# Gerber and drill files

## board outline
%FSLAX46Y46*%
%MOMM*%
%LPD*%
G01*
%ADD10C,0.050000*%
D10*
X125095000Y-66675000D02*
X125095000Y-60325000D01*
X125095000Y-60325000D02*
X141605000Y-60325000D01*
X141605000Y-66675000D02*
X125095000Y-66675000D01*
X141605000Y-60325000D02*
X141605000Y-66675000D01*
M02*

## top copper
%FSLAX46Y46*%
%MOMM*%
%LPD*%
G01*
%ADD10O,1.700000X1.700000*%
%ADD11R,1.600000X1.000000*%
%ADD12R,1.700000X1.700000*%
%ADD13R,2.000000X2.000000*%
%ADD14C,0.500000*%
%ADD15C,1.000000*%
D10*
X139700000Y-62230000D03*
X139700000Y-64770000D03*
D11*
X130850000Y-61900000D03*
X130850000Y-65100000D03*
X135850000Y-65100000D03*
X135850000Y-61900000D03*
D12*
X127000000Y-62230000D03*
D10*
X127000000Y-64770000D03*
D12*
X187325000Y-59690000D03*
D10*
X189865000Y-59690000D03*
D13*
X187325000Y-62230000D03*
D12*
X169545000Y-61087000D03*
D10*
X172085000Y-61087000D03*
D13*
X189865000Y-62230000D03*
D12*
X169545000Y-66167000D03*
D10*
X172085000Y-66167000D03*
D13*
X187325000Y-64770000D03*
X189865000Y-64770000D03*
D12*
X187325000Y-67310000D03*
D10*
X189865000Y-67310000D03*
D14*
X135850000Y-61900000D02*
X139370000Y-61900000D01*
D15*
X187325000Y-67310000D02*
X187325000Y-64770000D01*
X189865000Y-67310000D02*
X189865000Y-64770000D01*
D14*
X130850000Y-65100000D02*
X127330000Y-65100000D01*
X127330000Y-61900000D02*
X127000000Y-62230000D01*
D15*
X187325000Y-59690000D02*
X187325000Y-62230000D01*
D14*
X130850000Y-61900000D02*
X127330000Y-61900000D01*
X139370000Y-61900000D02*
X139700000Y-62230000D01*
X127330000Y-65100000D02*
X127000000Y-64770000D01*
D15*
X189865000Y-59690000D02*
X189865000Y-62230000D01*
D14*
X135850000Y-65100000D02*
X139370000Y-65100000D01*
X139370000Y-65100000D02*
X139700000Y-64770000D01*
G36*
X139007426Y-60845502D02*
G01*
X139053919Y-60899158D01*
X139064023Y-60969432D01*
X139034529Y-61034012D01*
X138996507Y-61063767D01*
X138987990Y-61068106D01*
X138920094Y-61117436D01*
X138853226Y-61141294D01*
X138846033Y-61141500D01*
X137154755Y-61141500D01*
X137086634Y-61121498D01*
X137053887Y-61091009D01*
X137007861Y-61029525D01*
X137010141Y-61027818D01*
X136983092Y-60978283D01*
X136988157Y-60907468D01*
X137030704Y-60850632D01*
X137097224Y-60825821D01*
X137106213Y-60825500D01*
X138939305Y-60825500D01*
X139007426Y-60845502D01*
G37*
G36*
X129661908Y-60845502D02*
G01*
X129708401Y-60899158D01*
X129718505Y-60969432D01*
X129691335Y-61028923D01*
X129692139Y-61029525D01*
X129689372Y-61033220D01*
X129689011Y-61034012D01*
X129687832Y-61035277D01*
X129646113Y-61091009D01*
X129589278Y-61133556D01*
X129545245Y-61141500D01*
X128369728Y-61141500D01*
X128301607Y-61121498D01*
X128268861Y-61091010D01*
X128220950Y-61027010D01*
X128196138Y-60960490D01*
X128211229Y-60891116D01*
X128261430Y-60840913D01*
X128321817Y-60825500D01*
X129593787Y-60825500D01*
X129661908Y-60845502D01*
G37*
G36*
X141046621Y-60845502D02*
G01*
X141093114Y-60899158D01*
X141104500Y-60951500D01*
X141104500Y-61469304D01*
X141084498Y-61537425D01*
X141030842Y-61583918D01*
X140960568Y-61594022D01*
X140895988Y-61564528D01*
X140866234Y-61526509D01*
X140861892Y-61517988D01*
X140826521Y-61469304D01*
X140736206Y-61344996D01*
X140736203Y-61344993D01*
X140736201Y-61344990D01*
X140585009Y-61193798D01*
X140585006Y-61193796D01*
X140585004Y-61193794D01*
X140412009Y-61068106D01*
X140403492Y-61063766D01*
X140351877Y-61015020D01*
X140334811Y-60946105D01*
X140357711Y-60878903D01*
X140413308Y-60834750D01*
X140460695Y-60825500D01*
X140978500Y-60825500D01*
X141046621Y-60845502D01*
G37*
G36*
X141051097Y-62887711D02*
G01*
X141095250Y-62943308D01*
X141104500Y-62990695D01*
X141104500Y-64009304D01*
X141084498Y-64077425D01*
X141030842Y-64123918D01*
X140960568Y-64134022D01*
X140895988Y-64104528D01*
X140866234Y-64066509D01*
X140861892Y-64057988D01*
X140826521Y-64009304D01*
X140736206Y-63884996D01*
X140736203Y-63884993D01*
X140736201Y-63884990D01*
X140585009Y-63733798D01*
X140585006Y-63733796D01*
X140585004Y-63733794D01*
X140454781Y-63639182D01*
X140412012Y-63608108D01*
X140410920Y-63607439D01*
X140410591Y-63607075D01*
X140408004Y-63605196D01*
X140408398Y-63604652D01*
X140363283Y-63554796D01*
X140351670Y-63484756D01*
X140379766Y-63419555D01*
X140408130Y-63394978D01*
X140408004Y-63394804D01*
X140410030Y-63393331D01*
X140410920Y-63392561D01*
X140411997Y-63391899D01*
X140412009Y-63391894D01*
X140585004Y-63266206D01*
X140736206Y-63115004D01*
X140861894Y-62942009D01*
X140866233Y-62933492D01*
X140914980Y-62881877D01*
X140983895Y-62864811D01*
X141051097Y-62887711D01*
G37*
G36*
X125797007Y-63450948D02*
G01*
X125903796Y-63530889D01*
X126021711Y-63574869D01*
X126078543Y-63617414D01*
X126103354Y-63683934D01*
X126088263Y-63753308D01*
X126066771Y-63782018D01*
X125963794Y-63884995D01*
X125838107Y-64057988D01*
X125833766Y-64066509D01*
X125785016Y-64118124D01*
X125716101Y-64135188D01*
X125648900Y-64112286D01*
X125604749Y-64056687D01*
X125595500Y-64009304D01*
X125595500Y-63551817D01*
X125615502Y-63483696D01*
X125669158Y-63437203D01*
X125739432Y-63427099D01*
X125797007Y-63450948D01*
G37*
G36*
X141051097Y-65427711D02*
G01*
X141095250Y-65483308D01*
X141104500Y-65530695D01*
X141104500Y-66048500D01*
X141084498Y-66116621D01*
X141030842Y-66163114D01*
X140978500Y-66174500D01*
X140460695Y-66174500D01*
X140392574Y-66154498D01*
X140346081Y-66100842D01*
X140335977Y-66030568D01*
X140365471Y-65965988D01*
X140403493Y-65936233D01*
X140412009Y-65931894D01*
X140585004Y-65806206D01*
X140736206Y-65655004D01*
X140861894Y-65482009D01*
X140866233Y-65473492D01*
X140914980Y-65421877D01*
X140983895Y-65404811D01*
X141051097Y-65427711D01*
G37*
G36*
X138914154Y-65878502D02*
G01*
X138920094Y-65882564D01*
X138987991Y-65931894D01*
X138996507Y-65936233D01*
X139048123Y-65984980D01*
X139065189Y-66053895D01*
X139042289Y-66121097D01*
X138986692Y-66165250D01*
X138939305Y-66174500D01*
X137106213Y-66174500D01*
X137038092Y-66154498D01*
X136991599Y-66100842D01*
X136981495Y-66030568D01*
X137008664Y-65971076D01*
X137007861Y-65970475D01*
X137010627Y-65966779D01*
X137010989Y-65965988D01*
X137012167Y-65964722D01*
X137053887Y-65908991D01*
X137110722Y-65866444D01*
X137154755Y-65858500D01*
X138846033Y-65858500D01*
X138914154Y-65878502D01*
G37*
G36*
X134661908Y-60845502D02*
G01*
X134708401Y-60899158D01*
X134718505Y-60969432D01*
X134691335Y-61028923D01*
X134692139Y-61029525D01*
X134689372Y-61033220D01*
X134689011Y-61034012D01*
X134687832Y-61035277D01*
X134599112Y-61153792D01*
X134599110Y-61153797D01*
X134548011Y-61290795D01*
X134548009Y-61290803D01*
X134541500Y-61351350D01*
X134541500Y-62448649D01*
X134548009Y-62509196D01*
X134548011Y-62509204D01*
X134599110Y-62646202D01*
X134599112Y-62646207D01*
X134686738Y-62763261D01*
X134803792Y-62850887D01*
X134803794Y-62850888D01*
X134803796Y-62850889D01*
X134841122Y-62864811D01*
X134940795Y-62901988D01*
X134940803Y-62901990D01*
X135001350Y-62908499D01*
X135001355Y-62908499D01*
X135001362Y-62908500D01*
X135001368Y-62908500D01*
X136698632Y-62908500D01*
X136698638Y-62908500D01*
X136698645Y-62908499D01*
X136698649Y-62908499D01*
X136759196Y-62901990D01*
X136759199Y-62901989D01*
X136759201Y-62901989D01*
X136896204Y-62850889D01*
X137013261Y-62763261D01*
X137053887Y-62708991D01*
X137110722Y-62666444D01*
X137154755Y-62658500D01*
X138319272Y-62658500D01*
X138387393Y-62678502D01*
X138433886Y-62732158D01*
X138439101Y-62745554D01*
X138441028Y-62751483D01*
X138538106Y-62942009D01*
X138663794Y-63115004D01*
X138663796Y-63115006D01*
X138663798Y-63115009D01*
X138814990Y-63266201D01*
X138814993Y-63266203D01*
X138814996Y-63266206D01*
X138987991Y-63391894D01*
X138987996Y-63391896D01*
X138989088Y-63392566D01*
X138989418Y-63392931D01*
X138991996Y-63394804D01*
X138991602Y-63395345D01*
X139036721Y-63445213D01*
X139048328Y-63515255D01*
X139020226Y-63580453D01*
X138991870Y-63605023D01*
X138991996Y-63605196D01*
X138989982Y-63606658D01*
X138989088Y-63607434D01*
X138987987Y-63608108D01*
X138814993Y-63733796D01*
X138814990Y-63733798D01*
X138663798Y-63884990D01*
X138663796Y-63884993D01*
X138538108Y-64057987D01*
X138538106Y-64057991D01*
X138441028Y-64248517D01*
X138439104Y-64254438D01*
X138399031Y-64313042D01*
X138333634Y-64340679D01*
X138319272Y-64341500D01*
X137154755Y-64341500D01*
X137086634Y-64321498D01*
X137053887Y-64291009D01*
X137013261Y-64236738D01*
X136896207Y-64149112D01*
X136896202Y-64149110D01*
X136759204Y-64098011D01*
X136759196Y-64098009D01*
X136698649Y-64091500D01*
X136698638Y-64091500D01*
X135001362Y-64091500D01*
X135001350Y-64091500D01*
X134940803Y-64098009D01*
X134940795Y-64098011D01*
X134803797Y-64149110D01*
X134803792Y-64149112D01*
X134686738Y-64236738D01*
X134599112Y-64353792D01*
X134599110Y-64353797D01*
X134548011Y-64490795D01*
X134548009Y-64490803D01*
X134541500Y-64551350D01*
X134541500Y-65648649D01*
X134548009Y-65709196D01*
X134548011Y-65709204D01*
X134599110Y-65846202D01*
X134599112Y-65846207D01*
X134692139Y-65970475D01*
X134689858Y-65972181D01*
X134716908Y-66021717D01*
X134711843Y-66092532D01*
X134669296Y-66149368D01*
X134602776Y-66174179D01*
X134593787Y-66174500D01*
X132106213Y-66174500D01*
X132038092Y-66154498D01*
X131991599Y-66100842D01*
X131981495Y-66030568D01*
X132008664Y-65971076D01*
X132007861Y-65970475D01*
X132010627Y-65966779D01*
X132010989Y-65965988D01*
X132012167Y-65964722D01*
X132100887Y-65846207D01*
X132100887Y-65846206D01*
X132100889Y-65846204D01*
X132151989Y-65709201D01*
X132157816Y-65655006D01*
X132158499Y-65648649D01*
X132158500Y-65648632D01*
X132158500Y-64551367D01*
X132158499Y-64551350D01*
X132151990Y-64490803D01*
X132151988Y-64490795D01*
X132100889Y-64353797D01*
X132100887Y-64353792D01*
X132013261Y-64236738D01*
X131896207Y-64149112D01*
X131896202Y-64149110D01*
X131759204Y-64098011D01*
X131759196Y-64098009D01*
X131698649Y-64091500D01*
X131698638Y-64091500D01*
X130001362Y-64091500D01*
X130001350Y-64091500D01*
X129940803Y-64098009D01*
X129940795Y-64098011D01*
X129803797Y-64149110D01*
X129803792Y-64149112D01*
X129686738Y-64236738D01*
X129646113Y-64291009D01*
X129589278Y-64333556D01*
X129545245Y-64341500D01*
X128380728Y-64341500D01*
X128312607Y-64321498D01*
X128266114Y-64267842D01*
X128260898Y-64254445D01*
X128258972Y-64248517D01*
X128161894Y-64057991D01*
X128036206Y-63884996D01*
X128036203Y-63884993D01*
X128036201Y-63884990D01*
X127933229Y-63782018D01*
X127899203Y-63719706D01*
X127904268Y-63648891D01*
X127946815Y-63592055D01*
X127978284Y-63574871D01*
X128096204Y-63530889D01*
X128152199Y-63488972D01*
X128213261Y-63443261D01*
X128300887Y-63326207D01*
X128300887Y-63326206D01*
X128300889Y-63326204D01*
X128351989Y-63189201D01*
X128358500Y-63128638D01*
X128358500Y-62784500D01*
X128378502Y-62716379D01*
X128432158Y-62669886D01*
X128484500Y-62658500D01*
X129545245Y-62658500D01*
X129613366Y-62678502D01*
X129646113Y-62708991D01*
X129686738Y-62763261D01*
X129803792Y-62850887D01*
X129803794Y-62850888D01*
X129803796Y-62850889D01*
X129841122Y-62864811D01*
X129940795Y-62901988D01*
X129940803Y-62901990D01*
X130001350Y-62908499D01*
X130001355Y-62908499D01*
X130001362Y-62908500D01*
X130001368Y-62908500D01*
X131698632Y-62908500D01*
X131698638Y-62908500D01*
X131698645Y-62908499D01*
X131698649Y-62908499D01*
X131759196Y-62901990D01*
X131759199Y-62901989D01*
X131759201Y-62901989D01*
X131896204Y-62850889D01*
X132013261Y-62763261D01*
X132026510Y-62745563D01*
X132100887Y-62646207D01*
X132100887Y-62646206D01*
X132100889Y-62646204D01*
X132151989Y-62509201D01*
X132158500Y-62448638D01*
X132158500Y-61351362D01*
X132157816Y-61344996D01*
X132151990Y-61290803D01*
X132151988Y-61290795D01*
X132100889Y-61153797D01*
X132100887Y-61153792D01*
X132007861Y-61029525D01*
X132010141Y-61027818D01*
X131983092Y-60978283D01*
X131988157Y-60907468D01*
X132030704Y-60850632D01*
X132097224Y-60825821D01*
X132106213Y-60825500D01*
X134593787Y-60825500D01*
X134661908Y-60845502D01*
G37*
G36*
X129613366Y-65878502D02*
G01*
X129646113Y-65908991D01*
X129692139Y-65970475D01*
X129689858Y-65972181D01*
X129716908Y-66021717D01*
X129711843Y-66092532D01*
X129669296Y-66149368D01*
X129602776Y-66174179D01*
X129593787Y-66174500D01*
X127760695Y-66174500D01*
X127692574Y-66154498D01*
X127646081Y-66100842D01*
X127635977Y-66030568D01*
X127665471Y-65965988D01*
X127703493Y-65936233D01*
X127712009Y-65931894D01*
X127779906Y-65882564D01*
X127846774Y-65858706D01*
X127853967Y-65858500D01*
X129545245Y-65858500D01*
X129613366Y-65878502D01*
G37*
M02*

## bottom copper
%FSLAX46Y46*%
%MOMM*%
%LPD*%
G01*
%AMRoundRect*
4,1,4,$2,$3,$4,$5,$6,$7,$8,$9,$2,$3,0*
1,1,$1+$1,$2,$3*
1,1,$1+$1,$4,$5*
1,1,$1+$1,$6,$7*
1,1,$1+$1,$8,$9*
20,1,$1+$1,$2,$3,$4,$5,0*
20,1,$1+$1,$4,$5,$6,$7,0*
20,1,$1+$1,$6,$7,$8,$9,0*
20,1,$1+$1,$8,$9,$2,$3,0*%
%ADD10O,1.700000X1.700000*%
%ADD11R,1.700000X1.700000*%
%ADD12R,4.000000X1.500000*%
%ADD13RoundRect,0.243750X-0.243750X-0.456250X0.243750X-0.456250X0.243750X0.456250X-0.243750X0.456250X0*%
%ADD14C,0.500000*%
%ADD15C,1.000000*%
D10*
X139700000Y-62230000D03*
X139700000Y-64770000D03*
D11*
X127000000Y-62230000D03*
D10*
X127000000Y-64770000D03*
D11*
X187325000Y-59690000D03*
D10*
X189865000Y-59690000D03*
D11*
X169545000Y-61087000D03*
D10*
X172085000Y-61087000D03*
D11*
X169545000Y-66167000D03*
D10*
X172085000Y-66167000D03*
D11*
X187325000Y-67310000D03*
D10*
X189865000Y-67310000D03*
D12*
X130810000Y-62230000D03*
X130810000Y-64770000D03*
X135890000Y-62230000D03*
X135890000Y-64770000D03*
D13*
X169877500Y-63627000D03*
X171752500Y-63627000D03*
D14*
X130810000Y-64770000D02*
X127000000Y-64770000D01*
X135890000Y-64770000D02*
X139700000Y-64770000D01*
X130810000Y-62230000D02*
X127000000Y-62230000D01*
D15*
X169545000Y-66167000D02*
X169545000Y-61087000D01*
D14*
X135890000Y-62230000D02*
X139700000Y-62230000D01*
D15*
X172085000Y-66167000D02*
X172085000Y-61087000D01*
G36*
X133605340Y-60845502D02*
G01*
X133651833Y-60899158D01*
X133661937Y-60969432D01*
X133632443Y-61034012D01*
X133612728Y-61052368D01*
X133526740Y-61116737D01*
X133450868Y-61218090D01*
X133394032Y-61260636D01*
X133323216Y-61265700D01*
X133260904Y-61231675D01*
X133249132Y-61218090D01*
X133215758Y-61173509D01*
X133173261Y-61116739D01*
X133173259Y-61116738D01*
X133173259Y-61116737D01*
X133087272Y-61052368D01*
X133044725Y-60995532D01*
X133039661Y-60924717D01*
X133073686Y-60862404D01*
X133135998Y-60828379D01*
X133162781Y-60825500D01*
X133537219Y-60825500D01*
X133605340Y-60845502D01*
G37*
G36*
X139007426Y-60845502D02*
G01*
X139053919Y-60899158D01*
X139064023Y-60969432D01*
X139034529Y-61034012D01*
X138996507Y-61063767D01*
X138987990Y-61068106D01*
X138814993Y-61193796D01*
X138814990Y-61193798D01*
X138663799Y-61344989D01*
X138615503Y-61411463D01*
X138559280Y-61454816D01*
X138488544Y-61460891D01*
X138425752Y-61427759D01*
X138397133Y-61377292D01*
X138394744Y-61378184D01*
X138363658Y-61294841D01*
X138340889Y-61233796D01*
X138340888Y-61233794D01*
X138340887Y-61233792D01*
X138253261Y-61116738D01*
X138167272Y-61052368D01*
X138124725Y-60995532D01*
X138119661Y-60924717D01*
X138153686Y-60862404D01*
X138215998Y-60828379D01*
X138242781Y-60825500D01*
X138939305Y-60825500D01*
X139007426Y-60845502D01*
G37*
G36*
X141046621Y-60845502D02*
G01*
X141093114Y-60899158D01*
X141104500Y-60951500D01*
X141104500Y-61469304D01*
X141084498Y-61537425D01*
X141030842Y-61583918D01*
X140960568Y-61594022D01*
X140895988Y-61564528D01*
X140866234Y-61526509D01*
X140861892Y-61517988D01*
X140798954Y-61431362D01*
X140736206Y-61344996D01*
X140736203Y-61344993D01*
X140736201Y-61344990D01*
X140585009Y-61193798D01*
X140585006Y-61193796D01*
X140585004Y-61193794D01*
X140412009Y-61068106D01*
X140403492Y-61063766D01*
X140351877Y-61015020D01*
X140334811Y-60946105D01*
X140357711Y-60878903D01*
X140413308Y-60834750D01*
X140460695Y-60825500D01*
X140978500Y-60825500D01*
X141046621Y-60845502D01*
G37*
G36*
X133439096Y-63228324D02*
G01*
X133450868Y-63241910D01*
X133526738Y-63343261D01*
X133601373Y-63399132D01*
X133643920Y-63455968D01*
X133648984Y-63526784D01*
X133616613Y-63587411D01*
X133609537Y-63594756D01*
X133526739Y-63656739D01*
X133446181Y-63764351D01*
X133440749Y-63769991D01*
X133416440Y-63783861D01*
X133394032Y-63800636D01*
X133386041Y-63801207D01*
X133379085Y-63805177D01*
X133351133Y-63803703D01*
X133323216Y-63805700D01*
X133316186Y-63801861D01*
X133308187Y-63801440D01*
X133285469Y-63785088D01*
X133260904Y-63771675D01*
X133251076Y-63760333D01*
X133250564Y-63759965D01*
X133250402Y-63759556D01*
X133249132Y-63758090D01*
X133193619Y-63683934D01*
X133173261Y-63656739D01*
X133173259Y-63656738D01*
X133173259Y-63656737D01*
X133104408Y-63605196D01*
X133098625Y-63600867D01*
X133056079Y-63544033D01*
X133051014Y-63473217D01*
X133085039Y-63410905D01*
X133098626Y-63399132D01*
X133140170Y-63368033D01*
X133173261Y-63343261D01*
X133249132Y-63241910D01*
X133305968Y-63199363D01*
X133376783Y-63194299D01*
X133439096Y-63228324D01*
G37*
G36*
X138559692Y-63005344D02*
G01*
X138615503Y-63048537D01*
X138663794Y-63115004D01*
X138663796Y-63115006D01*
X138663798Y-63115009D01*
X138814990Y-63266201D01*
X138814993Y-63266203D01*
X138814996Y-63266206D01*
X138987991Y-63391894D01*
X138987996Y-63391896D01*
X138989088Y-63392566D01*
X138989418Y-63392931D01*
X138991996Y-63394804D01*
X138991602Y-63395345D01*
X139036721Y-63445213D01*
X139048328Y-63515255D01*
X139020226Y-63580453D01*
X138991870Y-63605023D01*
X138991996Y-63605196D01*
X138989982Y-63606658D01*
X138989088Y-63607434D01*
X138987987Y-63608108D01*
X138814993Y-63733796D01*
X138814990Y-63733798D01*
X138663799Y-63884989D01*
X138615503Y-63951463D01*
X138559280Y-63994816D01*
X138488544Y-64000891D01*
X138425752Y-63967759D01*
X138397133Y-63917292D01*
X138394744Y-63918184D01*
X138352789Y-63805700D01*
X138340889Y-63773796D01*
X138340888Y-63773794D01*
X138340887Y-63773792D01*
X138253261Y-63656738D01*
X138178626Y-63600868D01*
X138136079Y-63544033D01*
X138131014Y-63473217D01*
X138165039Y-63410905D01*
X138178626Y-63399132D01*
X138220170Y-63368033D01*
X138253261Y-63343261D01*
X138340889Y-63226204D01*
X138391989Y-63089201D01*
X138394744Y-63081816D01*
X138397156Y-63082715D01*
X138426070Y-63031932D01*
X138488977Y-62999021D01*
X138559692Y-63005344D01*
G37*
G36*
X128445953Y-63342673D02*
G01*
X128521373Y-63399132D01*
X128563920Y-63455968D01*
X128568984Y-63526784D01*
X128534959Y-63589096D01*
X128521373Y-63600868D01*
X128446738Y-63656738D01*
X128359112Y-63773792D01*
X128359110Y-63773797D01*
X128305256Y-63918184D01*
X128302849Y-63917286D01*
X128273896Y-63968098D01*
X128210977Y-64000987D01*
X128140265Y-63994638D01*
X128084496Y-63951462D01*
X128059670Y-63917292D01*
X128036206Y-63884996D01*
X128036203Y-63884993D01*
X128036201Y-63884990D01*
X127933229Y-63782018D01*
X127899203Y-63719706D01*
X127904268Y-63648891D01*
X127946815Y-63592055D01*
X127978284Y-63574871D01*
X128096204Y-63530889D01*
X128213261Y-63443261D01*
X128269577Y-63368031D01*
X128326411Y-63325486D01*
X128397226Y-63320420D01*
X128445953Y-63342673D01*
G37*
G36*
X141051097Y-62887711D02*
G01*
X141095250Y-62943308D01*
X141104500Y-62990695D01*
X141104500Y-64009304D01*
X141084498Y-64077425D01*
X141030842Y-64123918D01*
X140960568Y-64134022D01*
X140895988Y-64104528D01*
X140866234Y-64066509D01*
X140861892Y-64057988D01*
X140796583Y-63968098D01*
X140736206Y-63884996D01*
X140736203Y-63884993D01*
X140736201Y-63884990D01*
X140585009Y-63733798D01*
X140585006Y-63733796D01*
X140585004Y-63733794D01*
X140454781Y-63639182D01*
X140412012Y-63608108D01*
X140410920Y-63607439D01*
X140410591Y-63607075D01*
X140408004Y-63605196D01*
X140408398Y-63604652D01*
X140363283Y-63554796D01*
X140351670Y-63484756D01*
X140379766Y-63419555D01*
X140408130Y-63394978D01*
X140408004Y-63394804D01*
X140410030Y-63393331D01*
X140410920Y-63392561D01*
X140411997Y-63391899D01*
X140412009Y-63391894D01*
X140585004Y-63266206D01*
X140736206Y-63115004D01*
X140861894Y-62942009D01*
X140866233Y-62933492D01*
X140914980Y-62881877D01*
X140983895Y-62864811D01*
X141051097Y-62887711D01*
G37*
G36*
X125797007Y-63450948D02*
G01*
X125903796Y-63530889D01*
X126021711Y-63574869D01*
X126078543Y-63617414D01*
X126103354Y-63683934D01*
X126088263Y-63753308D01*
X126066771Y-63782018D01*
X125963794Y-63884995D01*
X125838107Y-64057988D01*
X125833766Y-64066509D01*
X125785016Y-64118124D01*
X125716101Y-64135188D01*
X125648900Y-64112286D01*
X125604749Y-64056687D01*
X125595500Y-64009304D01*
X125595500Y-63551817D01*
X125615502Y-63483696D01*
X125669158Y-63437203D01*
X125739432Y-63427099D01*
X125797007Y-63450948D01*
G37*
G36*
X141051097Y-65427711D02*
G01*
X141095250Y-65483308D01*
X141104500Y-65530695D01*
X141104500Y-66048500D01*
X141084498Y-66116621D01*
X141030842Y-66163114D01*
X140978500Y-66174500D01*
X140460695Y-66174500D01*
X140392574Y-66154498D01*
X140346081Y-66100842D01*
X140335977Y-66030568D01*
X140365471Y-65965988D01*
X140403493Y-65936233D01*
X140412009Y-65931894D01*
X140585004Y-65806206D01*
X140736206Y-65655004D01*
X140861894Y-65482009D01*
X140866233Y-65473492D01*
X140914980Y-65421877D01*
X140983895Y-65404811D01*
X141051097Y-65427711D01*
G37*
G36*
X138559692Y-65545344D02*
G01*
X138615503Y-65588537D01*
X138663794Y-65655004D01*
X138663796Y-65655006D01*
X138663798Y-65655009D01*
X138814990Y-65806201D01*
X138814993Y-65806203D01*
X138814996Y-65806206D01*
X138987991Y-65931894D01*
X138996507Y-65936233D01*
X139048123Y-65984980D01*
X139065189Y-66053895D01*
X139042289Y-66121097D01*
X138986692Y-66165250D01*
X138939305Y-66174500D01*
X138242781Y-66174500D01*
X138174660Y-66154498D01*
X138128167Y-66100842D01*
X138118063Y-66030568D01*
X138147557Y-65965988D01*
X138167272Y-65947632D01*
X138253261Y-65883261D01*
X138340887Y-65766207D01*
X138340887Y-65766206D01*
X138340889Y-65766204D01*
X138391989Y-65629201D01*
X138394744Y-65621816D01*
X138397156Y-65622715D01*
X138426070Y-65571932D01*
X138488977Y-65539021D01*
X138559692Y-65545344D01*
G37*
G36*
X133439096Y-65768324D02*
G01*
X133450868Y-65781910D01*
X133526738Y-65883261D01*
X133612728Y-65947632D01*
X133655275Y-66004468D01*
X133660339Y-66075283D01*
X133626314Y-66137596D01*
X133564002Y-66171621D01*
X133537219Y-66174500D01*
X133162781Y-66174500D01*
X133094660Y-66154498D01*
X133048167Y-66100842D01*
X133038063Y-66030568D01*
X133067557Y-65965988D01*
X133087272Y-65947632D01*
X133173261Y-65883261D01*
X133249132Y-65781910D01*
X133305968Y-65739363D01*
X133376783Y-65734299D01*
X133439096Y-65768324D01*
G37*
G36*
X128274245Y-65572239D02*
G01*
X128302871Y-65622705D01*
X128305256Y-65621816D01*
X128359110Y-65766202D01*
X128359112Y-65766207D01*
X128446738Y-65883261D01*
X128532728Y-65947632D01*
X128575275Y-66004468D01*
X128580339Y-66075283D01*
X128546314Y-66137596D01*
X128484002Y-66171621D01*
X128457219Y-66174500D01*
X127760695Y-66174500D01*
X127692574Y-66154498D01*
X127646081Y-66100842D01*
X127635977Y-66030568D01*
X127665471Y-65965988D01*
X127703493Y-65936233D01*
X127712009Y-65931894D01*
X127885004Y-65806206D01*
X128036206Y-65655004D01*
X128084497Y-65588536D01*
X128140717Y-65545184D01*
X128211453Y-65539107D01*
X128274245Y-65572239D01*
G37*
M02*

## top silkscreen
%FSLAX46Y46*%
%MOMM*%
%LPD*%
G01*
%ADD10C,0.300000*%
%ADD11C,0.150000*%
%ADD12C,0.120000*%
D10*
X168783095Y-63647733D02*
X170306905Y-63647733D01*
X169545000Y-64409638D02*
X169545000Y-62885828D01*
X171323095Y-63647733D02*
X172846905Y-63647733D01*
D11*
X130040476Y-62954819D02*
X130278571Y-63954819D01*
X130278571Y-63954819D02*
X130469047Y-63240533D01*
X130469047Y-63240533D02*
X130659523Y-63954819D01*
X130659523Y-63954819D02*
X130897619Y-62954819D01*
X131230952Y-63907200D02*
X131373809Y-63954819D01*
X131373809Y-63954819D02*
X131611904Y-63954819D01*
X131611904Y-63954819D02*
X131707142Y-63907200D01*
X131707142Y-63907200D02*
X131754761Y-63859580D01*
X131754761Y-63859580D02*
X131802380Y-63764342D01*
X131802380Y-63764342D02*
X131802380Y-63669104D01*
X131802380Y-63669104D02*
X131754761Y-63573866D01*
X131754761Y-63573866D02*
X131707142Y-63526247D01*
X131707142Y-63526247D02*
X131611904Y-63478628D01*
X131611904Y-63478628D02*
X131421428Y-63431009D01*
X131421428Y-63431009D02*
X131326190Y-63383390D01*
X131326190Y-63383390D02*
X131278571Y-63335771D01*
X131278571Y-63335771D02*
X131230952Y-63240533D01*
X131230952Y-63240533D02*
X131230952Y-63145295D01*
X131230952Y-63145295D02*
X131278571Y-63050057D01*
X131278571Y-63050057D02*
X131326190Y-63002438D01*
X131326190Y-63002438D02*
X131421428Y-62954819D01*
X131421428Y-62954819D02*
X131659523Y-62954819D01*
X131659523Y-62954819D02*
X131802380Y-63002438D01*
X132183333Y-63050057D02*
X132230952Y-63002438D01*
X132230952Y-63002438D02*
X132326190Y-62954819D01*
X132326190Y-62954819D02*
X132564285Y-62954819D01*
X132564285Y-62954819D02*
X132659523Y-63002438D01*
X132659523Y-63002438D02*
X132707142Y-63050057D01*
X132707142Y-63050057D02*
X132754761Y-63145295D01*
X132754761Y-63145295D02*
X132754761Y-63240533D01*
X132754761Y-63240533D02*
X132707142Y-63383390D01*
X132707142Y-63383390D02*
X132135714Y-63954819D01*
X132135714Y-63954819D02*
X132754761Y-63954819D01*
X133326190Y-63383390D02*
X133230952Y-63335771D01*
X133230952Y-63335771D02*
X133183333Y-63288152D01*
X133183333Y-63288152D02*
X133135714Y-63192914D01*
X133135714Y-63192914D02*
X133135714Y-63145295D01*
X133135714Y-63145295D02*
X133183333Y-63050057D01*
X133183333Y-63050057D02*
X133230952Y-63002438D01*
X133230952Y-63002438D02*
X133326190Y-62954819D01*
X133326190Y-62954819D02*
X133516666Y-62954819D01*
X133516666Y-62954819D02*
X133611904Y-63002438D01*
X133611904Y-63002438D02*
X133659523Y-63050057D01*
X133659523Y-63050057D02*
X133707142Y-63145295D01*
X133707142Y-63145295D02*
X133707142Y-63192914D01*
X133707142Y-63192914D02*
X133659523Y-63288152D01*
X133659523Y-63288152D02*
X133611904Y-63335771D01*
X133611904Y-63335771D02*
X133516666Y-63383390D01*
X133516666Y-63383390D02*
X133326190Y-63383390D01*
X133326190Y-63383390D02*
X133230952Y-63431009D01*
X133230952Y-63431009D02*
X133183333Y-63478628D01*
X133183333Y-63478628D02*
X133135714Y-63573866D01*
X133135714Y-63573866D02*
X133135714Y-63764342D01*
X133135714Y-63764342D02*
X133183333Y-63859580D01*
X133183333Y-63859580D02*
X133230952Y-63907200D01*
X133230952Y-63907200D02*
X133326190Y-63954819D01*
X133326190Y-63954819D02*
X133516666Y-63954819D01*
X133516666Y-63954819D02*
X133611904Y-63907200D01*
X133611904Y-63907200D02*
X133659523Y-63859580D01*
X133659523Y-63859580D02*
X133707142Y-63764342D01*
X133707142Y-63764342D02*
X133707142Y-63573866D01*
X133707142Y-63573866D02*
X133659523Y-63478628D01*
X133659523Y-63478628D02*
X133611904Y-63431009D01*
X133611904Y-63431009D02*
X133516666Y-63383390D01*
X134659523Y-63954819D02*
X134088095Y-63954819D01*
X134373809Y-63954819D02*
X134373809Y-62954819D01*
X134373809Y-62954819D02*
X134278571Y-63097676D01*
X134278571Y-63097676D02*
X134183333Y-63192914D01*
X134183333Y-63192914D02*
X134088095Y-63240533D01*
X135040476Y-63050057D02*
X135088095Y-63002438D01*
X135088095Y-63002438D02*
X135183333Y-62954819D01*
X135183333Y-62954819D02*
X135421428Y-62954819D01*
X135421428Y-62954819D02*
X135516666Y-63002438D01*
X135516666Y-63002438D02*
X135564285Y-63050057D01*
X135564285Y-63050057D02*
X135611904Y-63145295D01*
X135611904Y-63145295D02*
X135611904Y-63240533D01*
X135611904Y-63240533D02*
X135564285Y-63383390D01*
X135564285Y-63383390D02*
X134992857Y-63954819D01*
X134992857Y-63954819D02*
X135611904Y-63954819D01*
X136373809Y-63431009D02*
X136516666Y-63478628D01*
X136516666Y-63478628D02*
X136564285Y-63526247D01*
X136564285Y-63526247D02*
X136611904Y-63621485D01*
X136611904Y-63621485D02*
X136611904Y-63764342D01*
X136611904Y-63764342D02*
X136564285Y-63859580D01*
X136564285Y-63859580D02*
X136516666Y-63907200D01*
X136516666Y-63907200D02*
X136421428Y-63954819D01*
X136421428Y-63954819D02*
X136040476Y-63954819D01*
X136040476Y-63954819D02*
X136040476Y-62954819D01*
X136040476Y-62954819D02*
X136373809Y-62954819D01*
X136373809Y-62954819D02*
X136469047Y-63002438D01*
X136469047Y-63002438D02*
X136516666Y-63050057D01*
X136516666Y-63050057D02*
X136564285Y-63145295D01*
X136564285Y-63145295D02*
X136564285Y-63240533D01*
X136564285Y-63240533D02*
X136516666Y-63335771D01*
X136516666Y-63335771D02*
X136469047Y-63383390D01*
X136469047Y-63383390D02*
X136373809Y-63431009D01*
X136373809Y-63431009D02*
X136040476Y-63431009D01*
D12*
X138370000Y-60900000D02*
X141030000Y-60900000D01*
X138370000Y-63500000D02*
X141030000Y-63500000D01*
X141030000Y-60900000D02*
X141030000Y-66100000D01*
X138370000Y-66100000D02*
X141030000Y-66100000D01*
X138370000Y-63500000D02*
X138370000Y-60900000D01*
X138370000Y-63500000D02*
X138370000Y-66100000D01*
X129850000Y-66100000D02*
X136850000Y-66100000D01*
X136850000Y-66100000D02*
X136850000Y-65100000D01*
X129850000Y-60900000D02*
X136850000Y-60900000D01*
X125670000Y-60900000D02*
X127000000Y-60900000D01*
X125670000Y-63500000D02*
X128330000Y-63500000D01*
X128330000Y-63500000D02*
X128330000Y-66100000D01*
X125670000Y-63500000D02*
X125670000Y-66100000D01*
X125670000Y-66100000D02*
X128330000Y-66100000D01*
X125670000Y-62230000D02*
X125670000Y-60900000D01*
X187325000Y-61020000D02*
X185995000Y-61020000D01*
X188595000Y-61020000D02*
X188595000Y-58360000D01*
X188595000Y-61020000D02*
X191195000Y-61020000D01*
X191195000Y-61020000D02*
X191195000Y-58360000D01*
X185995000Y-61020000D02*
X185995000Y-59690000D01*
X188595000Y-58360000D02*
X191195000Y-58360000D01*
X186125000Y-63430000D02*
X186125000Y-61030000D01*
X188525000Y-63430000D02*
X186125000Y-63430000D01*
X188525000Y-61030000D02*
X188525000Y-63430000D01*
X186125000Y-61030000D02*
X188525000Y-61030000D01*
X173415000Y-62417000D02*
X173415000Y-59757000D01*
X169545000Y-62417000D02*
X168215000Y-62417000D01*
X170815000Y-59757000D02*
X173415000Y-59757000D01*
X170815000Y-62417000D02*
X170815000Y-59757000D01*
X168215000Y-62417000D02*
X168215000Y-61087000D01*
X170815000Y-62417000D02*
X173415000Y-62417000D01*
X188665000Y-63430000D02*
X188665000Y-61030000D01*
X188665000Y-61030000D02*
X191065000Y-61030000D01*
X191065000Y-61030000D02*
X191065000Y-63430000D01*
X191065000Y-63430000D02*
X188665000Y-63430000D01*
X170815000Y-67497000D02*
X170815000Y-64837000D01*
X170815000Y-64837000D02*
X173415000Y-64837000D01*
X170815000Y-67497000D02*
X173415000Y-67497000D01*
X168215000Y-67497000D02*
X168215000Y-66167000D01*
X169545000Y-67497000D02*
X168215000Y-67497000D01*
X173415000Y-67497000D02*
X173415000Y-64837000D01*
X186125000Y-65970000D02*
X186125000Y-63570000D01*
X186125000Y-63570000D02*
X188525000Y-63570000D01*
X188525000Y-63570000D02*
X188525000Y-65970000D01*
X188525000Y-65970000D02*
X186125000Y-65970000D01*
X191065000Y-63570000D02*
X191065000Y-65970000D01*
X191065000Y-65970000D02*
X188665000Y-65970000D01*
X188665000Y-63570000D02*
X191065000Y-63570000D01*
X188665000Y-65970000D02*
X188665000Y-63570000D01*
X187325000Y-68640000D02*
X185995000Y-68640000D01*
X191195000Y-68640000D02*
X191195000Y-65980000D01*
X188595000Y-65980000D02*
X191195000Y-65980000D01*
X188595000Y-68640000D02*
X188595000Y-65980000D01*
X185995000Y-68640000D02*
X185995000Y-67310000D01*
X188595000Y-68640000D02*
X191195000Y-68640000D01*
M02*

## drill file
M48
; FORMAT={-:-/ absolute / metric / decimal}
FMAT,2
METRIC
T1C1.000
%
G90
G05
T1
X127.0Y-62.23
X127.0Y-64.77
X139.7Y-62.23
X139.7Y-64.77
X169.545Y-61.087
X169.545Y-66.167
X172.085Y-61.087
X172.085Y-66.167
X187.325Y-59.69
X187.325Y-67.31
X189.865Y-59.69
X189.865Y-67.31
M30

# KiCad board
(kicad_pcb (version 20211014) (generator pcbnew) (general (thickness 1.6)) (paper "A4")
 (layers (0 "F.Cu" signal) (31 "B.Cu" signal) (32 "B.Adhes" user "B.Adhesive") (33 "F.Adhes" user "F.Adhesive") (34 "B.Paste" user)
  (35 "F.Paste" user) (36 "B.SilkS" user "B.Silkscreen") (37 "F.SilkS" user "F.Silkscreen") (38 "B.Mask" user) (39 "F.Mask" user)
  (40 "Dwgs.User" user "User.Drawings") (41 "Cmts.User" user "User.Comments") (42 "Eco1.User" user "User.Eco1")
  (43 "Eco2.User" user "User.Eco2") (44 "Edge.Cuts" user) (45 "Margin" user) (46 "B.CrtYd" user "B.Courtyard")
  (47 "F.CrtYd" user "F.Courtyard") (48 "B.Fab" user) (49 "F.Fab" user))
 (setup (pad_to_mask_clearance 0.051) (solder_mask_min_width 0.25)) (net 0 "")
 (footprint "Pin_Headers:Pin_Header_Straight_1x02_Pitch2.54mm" (layer "F.Cu") (at 139.7 62.23)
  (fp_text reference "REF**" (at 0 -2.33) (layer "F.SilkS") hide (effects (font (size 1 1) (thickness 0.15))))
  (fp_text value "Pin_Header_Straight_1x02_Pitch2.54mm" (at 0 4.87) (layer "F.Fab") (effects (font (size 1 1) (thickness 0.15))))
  (fp_line (start -1.33 -1.33) (end 1.33 -1.33) (layer "F.SilkS") (width 0.12))
  (fp_line (start -1.33 1.27) (end 1.33 1.27) (layer "F.SilkS") (width 0.12))
  (fp_line (start 1.33 -1.33) (end 1.33 3.87) (layer "F.SilkS") (width 0.12))
  (fp_line (start -1.33 3.87) (end 1.33 3.87) (layer "F.SilkS") (width 0.12))
  (fp_line (start -1.33 1.27) (end -1.33 -1.33) (layer "F.SilkS") (width 0.12))
  (fp_line (start -1.33 1.27) (end -1.33 3.87) (layer "F.SilkS") (width 0.12))
  (pad "1" thru_hole oval locked (at 0 0) (size 1.7 1.7) (drill 1) (layers *.Cu *.Mask))
  (pad "2" thru_hole oval locked (at 0 2.54) (size 1.7 1.7) (drill 1) (layers *.Cu *.Mask)))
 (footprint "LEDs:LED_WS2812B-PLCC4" (layer "F.Cu") (at 133.35 63.5)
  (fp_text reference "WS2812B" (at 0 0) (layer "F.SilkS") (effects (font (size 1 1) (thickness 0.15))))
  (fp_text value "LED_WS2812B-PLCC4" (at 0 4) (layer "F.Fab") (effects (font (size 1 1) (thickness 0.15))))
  (fp_line (start -3.5 2.6) (end 3.5 2.6) (layer "F.SilkS") (width 0.12))
  (fp_line (start 3.5 2.6) (end 3.5 1.6) (layer "F.SilkS") (width 0.12))
  (fp_line (start -3.5 -2.6) (end 3.5 -2.6) (layer "F.SilkS") (width 0.12))
  (pad "1" smd rect locked (at -2.5 -1.6) (size 1.6 1) (layers "F.Cu" "F.Paste" "F.Mask"))
  (pad "2" smd rect locked (at -2.5 1.6) (size 1.6 1) (layers "F.Cu" "F.Paste" "F.Mask"))
  (pad "3" smd rect locked (at 2.5 1.6) (size 1.6 1) (layers "F.Cu" "F.Paste" "F.Mask"))
  (pad "4" smd rect locked (at 2.5 -1.6) (size 1.6 1) (layers "F.Cu" "F.Paste" "F.Mask")))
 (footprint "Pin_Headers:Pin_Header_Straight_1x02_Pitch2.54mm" (layer "F.Cu") (at 127 62.23)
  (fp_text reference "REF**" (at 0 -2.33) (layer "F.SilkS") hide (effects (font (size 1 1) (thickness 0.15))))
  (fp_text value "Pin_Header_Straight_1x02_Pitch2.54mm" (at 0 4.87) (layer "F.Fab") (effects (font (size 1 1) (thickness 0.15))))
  (fp_line (start -1.33 -1.33) (end 0 -1.33) (layer "F.SilkS") (width 0.12))
  (fp_line (start -1.33 1.27) (end 1.33 1.27) (layer "F.SilkS") (width 0.12))
  (fp_line (start 1.33 1.27) (end 1.33 3.87) (layer "F.SilkS") (width 0.12))
  (fp_line (start -1.33 1.27) (end -1.33 3.87) (layer "F.SilkS") (width 0.12))
  (fp_line (start -1.33 3.87) (end 1.33 3.87) (layer "F.SilkS") (width 0.12))
  (fp_line (start -1.33 0) (end -1.33 -1.33) (layer "F.SilkS") (width 0.12))
  (pad "1" thru_hole rect locked (at 0 0) (size 1.7 1.7) (drill 1) (layers *.Cu *.Mask))
  (pad "2" thru_hole oval locked (at 0 2.54) (size 1.7 1.7) (drill 1) (layers *.Cu *.Mask)))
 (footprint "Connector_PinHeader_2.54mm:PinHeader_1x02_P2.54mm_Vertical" (layer "F.Cu") (at 187.325 59.69 90)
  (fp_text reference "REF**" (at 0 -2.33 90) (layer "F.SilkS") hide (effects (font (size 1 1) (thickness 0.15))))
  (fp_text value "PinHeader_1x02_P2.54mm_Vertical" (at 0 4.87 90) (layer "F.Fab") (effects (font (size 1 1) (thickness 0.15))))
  (fp_line (start -1.33 0) (end -1.33 -1.33) (layer "F.SilkS") (width 0.12))
  (fp_line (start -1.33 1.27) (end 1.33 1.27) (layer "F.SilkS") (width 0.12))
  (fp_line (start -1.33 1.27) (end -1.33 3.87) (layer "F.SilkS") (width 0.12))
  (fp_line (start -1.33 3.87) (end 1.33 3.87) (layer "F.SilkS") (width 0.12))
  (fp_line (start -1.33 -1.33) (end 0 -1.33) (layer "F.SilkS") (width 0.12))
  (fp_line (start 1.33 1.27) (end 1.33 3.87) (layer "F.SilkS") (width 0.12))
  (pad "1" thru_hole rect locked (at 0 0 90) (size 1.7 1.7) (drill 1) (layers *.Cu *.Mask))
  (pad "2" thru_hole oval locked (at 0 2.54 90) (size 1.7 1.7) (drill 1) (layers *.Cu *.Mask)))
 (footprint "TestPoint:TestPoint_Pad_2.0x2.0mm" (layer "F.Cu") (at 187.325 62.23)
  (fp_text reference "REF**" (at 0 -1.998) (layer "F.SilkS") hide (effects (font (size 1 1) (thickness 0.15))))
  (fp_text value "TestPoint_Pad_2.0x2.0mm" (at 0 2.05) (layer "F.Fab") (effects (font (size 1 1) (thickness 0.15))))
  (fp_line (start -1.2 1.2) (end -1.2 -1.2) (layer "F.SilkS") (width 0.12))
  (fp_line (start 1.2 1.2) (end -1.2 1.2) (layer "F.SilkS") (width 0.12))
  (fp_line (start 1.2 -1.2) (end 1.2 1.2) (layer "F.SilkS") (width 0.12))
  (fp_line (start -1.2 -1.2) (end 1.2 -1.2) (layer "F.SilkS") (width 0.12))
  (pad "1" smd rect locked (at 0 0) (size 2 2) (layers "F.Cu" "F.Mask")))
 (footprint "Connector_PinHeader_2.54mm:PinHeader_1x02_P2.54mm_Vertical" (layer "F.Cu") (at 169.545 61.087 90)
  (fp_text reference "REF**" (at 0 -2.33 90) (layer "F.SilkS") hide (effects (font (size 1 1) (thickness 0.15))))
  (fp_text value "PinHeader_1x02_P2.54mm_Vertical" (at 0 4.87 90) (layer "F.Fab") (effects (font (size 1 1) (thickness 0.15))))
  (fp_line (start -1.33 3.87) (end 1.33 3.87) (layer "F.SilkS") (width 0.12))
  (fp_line (start -1.33 0) (end -1.33 -1.33) (layer "F.SilkS") (width 0.12))
  (fp_line (start 1.33 1.27) (end 1.33 3.87) (layer "F.SilkS") (width 0.12))
  (fp_line (start -1.33 1.27) (end 1.33 1.27) (layer "F.SilkS") (width 0.12))
  (fp_line (start -1.33 -1.33) (end 0 -1.33) (layer "F.SilkS") (width 0.12))
  (fp_line (start -1.33 1.27) (end -1.33 3.87) (layer "F.SilkS") (width 0.12))
  (pad "1" thru_hole rect locked (at 0 0 90) (size 1.7 1.7) (drill 1) (layers *.Cu *.Mask))
  (pad "2" thru_hole oval locked (at 0 2.54 90) (size 1.7 1.7) (drill 1) (layers *.Cu *.Mask)))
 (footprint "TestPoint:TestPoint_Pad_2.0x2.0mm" (layer "F.Cu") (at 189.865 62.23)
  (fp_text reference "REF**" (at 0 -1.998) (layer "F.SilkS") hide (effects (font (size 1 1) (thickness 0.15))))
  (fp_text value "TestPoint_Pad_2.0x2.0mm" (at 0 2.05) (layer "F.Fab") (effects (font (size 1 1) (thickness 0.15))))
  (fp_line (start -1.2 1.2) (end -1.2 -1.2) (layer "F.SilkS") (width 0.12))
  (fp_line (start -1.2 -1.2) (end 1.2 -1.2) (layer "F.SilkS") (width 0.12))
  (fp_line (start 1.2 -1.2) (end 1.2 1.2) (layer "F.SilkS") (width 0.12))
  (fp_line (start 1.2 1.2) (end -1.2 1.2) (layer "F.SilkS") (width 0.12))
  (pad "1" smd rect locked (at 0 0) (size 2 2) (layers "F.Cu" "F.Mask")))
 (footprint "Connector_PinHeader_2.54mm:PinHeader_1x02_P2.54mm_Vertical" (layer "F.Cu") (at 169.545 66.167 90)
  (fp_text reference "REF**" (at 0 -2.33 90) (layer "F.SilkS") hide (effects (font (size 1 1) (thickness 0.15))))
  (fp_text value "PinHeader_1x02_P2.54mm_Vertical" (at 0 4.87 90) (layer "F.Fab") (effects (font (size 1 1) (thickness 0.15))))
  (fp_line (start -1.33 1.27) (end 1.33 1.27) (layer "F.SilkS") (width 0.12))
  (fp_line (start 1.33 1.27) (end 1.33 3.87) (layer "F.SilkS") (width 0.12))
  (fp_line (start -1.33 1.27) (end -1.33 3.87) (layer "F.SilkS") (width 0.12))
  (fp_line (start -1.33 -1.33) (end 0 -1.33) (layer "F.SilkS") (width 0.12))
  (fp_line (start -1.33 0) (end -1.33 -1.33) (layer "F.SilkS") (width 0.12))
  (fp_line (start -1.33 3.87) (end 1.33 3.87) (layer "F.SilkS") (width 0.12))
  (pad "1" thru_hole rect locked (at 0 0 90) (size 1.7 1.7) (drill 1) (layers *.Cu *.Mask))
  (pad "2" thru_hole oval locked (at 0 2.54 90) (size 1.7 1.7) (drill 1) (layers *.Cu *.Mask)))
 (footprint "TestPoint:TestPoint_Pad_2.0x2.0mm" (layer "F.Cu") (at 187.325 64.77)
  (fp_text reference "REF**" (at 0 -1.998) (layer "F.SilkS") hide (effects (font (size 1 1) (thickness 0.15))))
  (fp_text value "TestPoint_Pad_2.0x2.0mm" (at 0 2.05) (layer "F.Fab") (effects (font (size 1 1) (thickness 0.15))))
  (fp_line (start -1.2 1.2) (end -1.2 -1.2) (layer "F.SilkS") (width 0.12))
  (fp_line (start -1.2 -1.2) (end 1.2 -1.2) (layer "F.SilkS") (width 0.12))
  (fp_line (start 1.2 -1.2) (end 1.2 1.2) (layer "F.SilkS") (width 0.12))
  (fp_line (start 1.2 1.2) (end -1.2 1.2) (layer "F.SilkS") (width 0.12))
  (pad "1" smd rect locked (at 0 0) (size 2 2) (layers "F.Cu" "F.Mask")))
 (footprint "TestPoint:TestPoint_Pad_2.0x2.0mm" (layer "F.Cu") (at 189.865 64.77)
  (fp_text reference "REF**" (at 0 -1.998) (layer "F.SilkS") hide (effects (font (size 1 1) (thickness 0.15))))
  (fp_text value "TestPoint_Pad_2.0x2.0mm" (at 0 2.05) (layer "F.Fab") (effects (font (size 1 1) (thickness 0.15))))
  (fp_line (start 1.2 -1.2) (end 1.2 1.2) (layer "F.SilkS") (width 0.12))
  (fp_line (start 1.2 1.2) (end -1.2 1.2) (layer "F.SilkS") (width 0.12))
  (fp_line (start -1.2 -1.2) (end 1.2 -1.2) (layer "F.SilkS") (width 0.12))
  (fp_line (start -1.2 1.2) (end -1.2 -1.2) (layer "F.SilkS") (width 0.12))
  (pad "1" smd rect locked (at 0 0) (size 2 2) (layers "F.Cu" "F.Mask")))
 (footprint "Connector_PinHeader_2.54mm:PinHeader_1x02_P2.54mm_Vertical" (layer "F.Cu") (at 187.325 67.31 90)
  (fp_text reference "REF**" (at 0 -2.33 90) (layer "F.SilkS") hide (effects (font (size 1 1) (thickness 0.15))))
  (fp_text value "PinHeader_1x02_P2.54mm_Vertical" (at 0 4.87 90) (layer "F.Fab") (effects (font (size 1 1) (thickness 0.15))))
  (fp_line (start -1.33 0) (end -1.33 -1.33) (layer "F.SilkS") (width 0.12))
  (fp_line (start -1.33 3.87) (end 1.33 3.87) (layer "F.SilkS") (width 0.12))
  (fp_line (start 1.33 1.27) (end 1.33 3.87) (layer "F.SilkS") (width 0.12))
  (fp_line (start -1.33 1.27) (end 1.33 1.27) (layer "F.SilkS") (width 0.12))
  (fp_line (start -1.33 -1.33) (end 0 -1.33) (layer "F.SilkS") (width 0.12))
  (fp_line (start -1.33 1.27) (end -1.33 3.87) (layer "F.SilkS") (width 0.12))
  (pad "1" thru_hole rect locked (at 0 0 90) (size 1.7 1.7) (drill 1) (layers *.Cu *.Mask))
  (pad "2" thru_hole oval locked (at 0 2.54 90) (size 1.7 1.7) (drill 1) (layers *.Cu *.Mask)))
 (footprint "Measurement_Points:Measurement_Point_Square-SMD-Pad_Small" (layer "B.Cu") (at 130.81 62.23)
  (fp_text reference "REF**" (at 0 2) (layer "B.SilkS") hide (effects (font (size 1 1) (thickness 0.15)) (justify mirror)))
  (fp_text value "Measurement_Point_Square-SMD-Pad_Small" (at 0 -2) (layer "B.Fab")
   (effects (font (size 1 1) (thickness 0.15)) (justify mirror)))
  (pad "1" smd rect locked (at 0 0) (size 4 1.5) (layers "B.Cu" "B.Mask")))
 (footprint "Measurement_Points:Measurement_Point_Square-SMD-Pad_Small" (layer "B.Cu") (at 130.81 64.77)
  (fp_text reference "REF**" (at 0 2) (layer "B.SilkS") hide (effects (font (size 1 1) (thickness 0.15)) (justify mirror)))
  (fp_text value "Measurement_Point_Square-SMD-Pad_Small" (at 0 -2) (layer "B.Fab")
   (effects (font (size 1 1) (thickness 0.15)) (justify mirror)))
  (pad "1" smd rect locked (at 0 0) (size 4 1.5) (layers "B.Cu" "B.Mask")))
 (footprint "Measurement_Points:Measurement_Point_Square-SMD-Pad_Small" (layer "B.Cu") (at 135.89 62.23)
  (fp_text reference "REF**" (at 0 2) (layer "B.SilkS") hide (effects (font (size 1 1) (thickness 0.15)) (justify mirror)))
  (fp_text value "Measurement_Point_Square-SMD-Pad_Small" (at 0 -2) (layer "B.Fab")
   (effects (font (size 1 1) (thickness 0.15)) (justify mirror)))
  (pad "1" smd rect locked (at 0 0) (size 4 1.5) (layers "B.Cu" "B.Mask")))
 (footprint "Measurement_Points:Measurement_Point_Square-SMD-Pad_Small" (layer "B.Cu") (at 135.89 64.77)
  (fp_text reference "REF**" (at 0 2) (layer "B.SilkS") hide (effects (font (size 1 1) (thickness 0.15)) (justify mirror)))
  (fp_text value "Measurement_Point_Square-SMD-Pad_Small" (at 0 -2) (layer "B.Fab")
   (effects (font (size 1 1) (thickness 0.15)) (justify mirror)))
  (pad "1" smd rect locked (at 0 0) (size 4 1.5) (layers "B.Cu" "B.Mask")))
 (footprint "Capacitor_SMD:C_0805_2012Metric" (layer "B.Cu") (at 170.815 63.627)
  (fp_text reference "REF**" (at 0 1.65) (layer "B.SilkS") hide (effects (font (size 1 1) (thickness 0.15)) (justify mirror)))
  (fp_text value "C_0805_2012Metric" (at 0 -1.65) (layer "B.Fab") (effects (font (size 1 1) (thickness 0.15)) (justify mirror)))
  (pad "1" smd roundrect locked (at -0.9375 0) (size 0.975 1.4) (layers "B.Cu" "B.Paste" "B.Mask") (roundrect_rratio 0.25))
  (pad "2" smd roundrect locked (at 0.9375 0) (size 0.975 1.4) (layers "B.Cu" "B.Paste" "B.Mask") (roundrect_rratio 0.25)))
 (gr_line (start 125.095 66.675) (end 125.095 60.325) (layer "Edge.Cuts") (width 0.05))
 (gr_line (start 125.095 60.325) (end 141.605 60.325) (layer "Edge.Cuts") (width 0.05))
 (gr_line (start 141.605 66.675) (end 125.095 66.675) (layer "Edge.Cuts") (width 0.05))
 (gr_line (start 141.605 60.325) (end 141.605 66.675) (layer "Edge.Cuts") (width 0.05))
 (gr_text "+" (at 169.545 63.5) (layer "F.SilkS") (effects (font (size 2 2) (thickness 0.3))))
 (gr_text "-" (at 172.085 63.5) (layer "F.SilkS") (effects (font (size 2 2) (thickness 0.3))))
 (segment (start 135.85 61.9) (end 139.37 61.9) (width 0.5) (layer "F.Cu") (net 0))
 (segment (start 187.325 67.31) (end 187.325 64.77) (width 1) (layer "F.Cu") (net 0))
 (segment (start 189.865 67.31) (end 189.865 64.77) (width 1) (layer "F.Cu") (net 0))
 (segment (start 130.85 65.1) (end 127.33 65.1) (width 0.5) (layer "F.Cu") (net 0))
 (segment (start 127.33 61.9) (end 127 62.23) (width 0.5) (layer "F.Cu") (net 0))
 (segment (start 187.325 59.69) (end 187.325 62.23) (width 1) (layer "F.Cu") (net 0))
 (segment (start 130.85 61.9) (end 127.33 61.9) (width 0.5) (layer "F.Cu") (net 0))
 (segment (start 139.37 61.9) (end 139.7 62.23) (width 0.5) (layer "F.Cu") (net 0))
 (segment (start 127.33 65.1) (end 127 64.77) (width 0.5) (layer "F.Cu") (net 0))
 (segment (start 189.865 59.69) (end 189.865 62.23) (width 1) (layer "F.Cu") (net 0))
 (segment (start 135.85 65.1) (end 139.37 65.1) (width 0.5) (layer "F.Cu") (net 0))
 (segment (start 139.37 65.1) (end 139.7 64.77) (width 0.5) (layer "F.Cu") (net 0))
 (segment (start 130.81 64.77) (end 127 64.77) (width 0.5) (layer "B.Cu") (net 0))
 (segment (start 135.89 64.77) (end 139.7 64.77) (width 0.5) (layer "B.Cu") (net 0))
 (segment (start 130.81 62.23) (end 127 62.23) (width 0.5) (layer "B.Cu") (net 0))
 (segment (start 169.545 66.167) (end 169.545 61.087) (width 1) (layer "B.Cu") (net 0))
 (segment (start 135.89 62.23) (end 139.7 62.23) (width 0.5) (layer "B.Cu") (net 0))
 (segment (start 172.085 66.167) (end 172.085 61.087) (width 1) (layer "B.Cu") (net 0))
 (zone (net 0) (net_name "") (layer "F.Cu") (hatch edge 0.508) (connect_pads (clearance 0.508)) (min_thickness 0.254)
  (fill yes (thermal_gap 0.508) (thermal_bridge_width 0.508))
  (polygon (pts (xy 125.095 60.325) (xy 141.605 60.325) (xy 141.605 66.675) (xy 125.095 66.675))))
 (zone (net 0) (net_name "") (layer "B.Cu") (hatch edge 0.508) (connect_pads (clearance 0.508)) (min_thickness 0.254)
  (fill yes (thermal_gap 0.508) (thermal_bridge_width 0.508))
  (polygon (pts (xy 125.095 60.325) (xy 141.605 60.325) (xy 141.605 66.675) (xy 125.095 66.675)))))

